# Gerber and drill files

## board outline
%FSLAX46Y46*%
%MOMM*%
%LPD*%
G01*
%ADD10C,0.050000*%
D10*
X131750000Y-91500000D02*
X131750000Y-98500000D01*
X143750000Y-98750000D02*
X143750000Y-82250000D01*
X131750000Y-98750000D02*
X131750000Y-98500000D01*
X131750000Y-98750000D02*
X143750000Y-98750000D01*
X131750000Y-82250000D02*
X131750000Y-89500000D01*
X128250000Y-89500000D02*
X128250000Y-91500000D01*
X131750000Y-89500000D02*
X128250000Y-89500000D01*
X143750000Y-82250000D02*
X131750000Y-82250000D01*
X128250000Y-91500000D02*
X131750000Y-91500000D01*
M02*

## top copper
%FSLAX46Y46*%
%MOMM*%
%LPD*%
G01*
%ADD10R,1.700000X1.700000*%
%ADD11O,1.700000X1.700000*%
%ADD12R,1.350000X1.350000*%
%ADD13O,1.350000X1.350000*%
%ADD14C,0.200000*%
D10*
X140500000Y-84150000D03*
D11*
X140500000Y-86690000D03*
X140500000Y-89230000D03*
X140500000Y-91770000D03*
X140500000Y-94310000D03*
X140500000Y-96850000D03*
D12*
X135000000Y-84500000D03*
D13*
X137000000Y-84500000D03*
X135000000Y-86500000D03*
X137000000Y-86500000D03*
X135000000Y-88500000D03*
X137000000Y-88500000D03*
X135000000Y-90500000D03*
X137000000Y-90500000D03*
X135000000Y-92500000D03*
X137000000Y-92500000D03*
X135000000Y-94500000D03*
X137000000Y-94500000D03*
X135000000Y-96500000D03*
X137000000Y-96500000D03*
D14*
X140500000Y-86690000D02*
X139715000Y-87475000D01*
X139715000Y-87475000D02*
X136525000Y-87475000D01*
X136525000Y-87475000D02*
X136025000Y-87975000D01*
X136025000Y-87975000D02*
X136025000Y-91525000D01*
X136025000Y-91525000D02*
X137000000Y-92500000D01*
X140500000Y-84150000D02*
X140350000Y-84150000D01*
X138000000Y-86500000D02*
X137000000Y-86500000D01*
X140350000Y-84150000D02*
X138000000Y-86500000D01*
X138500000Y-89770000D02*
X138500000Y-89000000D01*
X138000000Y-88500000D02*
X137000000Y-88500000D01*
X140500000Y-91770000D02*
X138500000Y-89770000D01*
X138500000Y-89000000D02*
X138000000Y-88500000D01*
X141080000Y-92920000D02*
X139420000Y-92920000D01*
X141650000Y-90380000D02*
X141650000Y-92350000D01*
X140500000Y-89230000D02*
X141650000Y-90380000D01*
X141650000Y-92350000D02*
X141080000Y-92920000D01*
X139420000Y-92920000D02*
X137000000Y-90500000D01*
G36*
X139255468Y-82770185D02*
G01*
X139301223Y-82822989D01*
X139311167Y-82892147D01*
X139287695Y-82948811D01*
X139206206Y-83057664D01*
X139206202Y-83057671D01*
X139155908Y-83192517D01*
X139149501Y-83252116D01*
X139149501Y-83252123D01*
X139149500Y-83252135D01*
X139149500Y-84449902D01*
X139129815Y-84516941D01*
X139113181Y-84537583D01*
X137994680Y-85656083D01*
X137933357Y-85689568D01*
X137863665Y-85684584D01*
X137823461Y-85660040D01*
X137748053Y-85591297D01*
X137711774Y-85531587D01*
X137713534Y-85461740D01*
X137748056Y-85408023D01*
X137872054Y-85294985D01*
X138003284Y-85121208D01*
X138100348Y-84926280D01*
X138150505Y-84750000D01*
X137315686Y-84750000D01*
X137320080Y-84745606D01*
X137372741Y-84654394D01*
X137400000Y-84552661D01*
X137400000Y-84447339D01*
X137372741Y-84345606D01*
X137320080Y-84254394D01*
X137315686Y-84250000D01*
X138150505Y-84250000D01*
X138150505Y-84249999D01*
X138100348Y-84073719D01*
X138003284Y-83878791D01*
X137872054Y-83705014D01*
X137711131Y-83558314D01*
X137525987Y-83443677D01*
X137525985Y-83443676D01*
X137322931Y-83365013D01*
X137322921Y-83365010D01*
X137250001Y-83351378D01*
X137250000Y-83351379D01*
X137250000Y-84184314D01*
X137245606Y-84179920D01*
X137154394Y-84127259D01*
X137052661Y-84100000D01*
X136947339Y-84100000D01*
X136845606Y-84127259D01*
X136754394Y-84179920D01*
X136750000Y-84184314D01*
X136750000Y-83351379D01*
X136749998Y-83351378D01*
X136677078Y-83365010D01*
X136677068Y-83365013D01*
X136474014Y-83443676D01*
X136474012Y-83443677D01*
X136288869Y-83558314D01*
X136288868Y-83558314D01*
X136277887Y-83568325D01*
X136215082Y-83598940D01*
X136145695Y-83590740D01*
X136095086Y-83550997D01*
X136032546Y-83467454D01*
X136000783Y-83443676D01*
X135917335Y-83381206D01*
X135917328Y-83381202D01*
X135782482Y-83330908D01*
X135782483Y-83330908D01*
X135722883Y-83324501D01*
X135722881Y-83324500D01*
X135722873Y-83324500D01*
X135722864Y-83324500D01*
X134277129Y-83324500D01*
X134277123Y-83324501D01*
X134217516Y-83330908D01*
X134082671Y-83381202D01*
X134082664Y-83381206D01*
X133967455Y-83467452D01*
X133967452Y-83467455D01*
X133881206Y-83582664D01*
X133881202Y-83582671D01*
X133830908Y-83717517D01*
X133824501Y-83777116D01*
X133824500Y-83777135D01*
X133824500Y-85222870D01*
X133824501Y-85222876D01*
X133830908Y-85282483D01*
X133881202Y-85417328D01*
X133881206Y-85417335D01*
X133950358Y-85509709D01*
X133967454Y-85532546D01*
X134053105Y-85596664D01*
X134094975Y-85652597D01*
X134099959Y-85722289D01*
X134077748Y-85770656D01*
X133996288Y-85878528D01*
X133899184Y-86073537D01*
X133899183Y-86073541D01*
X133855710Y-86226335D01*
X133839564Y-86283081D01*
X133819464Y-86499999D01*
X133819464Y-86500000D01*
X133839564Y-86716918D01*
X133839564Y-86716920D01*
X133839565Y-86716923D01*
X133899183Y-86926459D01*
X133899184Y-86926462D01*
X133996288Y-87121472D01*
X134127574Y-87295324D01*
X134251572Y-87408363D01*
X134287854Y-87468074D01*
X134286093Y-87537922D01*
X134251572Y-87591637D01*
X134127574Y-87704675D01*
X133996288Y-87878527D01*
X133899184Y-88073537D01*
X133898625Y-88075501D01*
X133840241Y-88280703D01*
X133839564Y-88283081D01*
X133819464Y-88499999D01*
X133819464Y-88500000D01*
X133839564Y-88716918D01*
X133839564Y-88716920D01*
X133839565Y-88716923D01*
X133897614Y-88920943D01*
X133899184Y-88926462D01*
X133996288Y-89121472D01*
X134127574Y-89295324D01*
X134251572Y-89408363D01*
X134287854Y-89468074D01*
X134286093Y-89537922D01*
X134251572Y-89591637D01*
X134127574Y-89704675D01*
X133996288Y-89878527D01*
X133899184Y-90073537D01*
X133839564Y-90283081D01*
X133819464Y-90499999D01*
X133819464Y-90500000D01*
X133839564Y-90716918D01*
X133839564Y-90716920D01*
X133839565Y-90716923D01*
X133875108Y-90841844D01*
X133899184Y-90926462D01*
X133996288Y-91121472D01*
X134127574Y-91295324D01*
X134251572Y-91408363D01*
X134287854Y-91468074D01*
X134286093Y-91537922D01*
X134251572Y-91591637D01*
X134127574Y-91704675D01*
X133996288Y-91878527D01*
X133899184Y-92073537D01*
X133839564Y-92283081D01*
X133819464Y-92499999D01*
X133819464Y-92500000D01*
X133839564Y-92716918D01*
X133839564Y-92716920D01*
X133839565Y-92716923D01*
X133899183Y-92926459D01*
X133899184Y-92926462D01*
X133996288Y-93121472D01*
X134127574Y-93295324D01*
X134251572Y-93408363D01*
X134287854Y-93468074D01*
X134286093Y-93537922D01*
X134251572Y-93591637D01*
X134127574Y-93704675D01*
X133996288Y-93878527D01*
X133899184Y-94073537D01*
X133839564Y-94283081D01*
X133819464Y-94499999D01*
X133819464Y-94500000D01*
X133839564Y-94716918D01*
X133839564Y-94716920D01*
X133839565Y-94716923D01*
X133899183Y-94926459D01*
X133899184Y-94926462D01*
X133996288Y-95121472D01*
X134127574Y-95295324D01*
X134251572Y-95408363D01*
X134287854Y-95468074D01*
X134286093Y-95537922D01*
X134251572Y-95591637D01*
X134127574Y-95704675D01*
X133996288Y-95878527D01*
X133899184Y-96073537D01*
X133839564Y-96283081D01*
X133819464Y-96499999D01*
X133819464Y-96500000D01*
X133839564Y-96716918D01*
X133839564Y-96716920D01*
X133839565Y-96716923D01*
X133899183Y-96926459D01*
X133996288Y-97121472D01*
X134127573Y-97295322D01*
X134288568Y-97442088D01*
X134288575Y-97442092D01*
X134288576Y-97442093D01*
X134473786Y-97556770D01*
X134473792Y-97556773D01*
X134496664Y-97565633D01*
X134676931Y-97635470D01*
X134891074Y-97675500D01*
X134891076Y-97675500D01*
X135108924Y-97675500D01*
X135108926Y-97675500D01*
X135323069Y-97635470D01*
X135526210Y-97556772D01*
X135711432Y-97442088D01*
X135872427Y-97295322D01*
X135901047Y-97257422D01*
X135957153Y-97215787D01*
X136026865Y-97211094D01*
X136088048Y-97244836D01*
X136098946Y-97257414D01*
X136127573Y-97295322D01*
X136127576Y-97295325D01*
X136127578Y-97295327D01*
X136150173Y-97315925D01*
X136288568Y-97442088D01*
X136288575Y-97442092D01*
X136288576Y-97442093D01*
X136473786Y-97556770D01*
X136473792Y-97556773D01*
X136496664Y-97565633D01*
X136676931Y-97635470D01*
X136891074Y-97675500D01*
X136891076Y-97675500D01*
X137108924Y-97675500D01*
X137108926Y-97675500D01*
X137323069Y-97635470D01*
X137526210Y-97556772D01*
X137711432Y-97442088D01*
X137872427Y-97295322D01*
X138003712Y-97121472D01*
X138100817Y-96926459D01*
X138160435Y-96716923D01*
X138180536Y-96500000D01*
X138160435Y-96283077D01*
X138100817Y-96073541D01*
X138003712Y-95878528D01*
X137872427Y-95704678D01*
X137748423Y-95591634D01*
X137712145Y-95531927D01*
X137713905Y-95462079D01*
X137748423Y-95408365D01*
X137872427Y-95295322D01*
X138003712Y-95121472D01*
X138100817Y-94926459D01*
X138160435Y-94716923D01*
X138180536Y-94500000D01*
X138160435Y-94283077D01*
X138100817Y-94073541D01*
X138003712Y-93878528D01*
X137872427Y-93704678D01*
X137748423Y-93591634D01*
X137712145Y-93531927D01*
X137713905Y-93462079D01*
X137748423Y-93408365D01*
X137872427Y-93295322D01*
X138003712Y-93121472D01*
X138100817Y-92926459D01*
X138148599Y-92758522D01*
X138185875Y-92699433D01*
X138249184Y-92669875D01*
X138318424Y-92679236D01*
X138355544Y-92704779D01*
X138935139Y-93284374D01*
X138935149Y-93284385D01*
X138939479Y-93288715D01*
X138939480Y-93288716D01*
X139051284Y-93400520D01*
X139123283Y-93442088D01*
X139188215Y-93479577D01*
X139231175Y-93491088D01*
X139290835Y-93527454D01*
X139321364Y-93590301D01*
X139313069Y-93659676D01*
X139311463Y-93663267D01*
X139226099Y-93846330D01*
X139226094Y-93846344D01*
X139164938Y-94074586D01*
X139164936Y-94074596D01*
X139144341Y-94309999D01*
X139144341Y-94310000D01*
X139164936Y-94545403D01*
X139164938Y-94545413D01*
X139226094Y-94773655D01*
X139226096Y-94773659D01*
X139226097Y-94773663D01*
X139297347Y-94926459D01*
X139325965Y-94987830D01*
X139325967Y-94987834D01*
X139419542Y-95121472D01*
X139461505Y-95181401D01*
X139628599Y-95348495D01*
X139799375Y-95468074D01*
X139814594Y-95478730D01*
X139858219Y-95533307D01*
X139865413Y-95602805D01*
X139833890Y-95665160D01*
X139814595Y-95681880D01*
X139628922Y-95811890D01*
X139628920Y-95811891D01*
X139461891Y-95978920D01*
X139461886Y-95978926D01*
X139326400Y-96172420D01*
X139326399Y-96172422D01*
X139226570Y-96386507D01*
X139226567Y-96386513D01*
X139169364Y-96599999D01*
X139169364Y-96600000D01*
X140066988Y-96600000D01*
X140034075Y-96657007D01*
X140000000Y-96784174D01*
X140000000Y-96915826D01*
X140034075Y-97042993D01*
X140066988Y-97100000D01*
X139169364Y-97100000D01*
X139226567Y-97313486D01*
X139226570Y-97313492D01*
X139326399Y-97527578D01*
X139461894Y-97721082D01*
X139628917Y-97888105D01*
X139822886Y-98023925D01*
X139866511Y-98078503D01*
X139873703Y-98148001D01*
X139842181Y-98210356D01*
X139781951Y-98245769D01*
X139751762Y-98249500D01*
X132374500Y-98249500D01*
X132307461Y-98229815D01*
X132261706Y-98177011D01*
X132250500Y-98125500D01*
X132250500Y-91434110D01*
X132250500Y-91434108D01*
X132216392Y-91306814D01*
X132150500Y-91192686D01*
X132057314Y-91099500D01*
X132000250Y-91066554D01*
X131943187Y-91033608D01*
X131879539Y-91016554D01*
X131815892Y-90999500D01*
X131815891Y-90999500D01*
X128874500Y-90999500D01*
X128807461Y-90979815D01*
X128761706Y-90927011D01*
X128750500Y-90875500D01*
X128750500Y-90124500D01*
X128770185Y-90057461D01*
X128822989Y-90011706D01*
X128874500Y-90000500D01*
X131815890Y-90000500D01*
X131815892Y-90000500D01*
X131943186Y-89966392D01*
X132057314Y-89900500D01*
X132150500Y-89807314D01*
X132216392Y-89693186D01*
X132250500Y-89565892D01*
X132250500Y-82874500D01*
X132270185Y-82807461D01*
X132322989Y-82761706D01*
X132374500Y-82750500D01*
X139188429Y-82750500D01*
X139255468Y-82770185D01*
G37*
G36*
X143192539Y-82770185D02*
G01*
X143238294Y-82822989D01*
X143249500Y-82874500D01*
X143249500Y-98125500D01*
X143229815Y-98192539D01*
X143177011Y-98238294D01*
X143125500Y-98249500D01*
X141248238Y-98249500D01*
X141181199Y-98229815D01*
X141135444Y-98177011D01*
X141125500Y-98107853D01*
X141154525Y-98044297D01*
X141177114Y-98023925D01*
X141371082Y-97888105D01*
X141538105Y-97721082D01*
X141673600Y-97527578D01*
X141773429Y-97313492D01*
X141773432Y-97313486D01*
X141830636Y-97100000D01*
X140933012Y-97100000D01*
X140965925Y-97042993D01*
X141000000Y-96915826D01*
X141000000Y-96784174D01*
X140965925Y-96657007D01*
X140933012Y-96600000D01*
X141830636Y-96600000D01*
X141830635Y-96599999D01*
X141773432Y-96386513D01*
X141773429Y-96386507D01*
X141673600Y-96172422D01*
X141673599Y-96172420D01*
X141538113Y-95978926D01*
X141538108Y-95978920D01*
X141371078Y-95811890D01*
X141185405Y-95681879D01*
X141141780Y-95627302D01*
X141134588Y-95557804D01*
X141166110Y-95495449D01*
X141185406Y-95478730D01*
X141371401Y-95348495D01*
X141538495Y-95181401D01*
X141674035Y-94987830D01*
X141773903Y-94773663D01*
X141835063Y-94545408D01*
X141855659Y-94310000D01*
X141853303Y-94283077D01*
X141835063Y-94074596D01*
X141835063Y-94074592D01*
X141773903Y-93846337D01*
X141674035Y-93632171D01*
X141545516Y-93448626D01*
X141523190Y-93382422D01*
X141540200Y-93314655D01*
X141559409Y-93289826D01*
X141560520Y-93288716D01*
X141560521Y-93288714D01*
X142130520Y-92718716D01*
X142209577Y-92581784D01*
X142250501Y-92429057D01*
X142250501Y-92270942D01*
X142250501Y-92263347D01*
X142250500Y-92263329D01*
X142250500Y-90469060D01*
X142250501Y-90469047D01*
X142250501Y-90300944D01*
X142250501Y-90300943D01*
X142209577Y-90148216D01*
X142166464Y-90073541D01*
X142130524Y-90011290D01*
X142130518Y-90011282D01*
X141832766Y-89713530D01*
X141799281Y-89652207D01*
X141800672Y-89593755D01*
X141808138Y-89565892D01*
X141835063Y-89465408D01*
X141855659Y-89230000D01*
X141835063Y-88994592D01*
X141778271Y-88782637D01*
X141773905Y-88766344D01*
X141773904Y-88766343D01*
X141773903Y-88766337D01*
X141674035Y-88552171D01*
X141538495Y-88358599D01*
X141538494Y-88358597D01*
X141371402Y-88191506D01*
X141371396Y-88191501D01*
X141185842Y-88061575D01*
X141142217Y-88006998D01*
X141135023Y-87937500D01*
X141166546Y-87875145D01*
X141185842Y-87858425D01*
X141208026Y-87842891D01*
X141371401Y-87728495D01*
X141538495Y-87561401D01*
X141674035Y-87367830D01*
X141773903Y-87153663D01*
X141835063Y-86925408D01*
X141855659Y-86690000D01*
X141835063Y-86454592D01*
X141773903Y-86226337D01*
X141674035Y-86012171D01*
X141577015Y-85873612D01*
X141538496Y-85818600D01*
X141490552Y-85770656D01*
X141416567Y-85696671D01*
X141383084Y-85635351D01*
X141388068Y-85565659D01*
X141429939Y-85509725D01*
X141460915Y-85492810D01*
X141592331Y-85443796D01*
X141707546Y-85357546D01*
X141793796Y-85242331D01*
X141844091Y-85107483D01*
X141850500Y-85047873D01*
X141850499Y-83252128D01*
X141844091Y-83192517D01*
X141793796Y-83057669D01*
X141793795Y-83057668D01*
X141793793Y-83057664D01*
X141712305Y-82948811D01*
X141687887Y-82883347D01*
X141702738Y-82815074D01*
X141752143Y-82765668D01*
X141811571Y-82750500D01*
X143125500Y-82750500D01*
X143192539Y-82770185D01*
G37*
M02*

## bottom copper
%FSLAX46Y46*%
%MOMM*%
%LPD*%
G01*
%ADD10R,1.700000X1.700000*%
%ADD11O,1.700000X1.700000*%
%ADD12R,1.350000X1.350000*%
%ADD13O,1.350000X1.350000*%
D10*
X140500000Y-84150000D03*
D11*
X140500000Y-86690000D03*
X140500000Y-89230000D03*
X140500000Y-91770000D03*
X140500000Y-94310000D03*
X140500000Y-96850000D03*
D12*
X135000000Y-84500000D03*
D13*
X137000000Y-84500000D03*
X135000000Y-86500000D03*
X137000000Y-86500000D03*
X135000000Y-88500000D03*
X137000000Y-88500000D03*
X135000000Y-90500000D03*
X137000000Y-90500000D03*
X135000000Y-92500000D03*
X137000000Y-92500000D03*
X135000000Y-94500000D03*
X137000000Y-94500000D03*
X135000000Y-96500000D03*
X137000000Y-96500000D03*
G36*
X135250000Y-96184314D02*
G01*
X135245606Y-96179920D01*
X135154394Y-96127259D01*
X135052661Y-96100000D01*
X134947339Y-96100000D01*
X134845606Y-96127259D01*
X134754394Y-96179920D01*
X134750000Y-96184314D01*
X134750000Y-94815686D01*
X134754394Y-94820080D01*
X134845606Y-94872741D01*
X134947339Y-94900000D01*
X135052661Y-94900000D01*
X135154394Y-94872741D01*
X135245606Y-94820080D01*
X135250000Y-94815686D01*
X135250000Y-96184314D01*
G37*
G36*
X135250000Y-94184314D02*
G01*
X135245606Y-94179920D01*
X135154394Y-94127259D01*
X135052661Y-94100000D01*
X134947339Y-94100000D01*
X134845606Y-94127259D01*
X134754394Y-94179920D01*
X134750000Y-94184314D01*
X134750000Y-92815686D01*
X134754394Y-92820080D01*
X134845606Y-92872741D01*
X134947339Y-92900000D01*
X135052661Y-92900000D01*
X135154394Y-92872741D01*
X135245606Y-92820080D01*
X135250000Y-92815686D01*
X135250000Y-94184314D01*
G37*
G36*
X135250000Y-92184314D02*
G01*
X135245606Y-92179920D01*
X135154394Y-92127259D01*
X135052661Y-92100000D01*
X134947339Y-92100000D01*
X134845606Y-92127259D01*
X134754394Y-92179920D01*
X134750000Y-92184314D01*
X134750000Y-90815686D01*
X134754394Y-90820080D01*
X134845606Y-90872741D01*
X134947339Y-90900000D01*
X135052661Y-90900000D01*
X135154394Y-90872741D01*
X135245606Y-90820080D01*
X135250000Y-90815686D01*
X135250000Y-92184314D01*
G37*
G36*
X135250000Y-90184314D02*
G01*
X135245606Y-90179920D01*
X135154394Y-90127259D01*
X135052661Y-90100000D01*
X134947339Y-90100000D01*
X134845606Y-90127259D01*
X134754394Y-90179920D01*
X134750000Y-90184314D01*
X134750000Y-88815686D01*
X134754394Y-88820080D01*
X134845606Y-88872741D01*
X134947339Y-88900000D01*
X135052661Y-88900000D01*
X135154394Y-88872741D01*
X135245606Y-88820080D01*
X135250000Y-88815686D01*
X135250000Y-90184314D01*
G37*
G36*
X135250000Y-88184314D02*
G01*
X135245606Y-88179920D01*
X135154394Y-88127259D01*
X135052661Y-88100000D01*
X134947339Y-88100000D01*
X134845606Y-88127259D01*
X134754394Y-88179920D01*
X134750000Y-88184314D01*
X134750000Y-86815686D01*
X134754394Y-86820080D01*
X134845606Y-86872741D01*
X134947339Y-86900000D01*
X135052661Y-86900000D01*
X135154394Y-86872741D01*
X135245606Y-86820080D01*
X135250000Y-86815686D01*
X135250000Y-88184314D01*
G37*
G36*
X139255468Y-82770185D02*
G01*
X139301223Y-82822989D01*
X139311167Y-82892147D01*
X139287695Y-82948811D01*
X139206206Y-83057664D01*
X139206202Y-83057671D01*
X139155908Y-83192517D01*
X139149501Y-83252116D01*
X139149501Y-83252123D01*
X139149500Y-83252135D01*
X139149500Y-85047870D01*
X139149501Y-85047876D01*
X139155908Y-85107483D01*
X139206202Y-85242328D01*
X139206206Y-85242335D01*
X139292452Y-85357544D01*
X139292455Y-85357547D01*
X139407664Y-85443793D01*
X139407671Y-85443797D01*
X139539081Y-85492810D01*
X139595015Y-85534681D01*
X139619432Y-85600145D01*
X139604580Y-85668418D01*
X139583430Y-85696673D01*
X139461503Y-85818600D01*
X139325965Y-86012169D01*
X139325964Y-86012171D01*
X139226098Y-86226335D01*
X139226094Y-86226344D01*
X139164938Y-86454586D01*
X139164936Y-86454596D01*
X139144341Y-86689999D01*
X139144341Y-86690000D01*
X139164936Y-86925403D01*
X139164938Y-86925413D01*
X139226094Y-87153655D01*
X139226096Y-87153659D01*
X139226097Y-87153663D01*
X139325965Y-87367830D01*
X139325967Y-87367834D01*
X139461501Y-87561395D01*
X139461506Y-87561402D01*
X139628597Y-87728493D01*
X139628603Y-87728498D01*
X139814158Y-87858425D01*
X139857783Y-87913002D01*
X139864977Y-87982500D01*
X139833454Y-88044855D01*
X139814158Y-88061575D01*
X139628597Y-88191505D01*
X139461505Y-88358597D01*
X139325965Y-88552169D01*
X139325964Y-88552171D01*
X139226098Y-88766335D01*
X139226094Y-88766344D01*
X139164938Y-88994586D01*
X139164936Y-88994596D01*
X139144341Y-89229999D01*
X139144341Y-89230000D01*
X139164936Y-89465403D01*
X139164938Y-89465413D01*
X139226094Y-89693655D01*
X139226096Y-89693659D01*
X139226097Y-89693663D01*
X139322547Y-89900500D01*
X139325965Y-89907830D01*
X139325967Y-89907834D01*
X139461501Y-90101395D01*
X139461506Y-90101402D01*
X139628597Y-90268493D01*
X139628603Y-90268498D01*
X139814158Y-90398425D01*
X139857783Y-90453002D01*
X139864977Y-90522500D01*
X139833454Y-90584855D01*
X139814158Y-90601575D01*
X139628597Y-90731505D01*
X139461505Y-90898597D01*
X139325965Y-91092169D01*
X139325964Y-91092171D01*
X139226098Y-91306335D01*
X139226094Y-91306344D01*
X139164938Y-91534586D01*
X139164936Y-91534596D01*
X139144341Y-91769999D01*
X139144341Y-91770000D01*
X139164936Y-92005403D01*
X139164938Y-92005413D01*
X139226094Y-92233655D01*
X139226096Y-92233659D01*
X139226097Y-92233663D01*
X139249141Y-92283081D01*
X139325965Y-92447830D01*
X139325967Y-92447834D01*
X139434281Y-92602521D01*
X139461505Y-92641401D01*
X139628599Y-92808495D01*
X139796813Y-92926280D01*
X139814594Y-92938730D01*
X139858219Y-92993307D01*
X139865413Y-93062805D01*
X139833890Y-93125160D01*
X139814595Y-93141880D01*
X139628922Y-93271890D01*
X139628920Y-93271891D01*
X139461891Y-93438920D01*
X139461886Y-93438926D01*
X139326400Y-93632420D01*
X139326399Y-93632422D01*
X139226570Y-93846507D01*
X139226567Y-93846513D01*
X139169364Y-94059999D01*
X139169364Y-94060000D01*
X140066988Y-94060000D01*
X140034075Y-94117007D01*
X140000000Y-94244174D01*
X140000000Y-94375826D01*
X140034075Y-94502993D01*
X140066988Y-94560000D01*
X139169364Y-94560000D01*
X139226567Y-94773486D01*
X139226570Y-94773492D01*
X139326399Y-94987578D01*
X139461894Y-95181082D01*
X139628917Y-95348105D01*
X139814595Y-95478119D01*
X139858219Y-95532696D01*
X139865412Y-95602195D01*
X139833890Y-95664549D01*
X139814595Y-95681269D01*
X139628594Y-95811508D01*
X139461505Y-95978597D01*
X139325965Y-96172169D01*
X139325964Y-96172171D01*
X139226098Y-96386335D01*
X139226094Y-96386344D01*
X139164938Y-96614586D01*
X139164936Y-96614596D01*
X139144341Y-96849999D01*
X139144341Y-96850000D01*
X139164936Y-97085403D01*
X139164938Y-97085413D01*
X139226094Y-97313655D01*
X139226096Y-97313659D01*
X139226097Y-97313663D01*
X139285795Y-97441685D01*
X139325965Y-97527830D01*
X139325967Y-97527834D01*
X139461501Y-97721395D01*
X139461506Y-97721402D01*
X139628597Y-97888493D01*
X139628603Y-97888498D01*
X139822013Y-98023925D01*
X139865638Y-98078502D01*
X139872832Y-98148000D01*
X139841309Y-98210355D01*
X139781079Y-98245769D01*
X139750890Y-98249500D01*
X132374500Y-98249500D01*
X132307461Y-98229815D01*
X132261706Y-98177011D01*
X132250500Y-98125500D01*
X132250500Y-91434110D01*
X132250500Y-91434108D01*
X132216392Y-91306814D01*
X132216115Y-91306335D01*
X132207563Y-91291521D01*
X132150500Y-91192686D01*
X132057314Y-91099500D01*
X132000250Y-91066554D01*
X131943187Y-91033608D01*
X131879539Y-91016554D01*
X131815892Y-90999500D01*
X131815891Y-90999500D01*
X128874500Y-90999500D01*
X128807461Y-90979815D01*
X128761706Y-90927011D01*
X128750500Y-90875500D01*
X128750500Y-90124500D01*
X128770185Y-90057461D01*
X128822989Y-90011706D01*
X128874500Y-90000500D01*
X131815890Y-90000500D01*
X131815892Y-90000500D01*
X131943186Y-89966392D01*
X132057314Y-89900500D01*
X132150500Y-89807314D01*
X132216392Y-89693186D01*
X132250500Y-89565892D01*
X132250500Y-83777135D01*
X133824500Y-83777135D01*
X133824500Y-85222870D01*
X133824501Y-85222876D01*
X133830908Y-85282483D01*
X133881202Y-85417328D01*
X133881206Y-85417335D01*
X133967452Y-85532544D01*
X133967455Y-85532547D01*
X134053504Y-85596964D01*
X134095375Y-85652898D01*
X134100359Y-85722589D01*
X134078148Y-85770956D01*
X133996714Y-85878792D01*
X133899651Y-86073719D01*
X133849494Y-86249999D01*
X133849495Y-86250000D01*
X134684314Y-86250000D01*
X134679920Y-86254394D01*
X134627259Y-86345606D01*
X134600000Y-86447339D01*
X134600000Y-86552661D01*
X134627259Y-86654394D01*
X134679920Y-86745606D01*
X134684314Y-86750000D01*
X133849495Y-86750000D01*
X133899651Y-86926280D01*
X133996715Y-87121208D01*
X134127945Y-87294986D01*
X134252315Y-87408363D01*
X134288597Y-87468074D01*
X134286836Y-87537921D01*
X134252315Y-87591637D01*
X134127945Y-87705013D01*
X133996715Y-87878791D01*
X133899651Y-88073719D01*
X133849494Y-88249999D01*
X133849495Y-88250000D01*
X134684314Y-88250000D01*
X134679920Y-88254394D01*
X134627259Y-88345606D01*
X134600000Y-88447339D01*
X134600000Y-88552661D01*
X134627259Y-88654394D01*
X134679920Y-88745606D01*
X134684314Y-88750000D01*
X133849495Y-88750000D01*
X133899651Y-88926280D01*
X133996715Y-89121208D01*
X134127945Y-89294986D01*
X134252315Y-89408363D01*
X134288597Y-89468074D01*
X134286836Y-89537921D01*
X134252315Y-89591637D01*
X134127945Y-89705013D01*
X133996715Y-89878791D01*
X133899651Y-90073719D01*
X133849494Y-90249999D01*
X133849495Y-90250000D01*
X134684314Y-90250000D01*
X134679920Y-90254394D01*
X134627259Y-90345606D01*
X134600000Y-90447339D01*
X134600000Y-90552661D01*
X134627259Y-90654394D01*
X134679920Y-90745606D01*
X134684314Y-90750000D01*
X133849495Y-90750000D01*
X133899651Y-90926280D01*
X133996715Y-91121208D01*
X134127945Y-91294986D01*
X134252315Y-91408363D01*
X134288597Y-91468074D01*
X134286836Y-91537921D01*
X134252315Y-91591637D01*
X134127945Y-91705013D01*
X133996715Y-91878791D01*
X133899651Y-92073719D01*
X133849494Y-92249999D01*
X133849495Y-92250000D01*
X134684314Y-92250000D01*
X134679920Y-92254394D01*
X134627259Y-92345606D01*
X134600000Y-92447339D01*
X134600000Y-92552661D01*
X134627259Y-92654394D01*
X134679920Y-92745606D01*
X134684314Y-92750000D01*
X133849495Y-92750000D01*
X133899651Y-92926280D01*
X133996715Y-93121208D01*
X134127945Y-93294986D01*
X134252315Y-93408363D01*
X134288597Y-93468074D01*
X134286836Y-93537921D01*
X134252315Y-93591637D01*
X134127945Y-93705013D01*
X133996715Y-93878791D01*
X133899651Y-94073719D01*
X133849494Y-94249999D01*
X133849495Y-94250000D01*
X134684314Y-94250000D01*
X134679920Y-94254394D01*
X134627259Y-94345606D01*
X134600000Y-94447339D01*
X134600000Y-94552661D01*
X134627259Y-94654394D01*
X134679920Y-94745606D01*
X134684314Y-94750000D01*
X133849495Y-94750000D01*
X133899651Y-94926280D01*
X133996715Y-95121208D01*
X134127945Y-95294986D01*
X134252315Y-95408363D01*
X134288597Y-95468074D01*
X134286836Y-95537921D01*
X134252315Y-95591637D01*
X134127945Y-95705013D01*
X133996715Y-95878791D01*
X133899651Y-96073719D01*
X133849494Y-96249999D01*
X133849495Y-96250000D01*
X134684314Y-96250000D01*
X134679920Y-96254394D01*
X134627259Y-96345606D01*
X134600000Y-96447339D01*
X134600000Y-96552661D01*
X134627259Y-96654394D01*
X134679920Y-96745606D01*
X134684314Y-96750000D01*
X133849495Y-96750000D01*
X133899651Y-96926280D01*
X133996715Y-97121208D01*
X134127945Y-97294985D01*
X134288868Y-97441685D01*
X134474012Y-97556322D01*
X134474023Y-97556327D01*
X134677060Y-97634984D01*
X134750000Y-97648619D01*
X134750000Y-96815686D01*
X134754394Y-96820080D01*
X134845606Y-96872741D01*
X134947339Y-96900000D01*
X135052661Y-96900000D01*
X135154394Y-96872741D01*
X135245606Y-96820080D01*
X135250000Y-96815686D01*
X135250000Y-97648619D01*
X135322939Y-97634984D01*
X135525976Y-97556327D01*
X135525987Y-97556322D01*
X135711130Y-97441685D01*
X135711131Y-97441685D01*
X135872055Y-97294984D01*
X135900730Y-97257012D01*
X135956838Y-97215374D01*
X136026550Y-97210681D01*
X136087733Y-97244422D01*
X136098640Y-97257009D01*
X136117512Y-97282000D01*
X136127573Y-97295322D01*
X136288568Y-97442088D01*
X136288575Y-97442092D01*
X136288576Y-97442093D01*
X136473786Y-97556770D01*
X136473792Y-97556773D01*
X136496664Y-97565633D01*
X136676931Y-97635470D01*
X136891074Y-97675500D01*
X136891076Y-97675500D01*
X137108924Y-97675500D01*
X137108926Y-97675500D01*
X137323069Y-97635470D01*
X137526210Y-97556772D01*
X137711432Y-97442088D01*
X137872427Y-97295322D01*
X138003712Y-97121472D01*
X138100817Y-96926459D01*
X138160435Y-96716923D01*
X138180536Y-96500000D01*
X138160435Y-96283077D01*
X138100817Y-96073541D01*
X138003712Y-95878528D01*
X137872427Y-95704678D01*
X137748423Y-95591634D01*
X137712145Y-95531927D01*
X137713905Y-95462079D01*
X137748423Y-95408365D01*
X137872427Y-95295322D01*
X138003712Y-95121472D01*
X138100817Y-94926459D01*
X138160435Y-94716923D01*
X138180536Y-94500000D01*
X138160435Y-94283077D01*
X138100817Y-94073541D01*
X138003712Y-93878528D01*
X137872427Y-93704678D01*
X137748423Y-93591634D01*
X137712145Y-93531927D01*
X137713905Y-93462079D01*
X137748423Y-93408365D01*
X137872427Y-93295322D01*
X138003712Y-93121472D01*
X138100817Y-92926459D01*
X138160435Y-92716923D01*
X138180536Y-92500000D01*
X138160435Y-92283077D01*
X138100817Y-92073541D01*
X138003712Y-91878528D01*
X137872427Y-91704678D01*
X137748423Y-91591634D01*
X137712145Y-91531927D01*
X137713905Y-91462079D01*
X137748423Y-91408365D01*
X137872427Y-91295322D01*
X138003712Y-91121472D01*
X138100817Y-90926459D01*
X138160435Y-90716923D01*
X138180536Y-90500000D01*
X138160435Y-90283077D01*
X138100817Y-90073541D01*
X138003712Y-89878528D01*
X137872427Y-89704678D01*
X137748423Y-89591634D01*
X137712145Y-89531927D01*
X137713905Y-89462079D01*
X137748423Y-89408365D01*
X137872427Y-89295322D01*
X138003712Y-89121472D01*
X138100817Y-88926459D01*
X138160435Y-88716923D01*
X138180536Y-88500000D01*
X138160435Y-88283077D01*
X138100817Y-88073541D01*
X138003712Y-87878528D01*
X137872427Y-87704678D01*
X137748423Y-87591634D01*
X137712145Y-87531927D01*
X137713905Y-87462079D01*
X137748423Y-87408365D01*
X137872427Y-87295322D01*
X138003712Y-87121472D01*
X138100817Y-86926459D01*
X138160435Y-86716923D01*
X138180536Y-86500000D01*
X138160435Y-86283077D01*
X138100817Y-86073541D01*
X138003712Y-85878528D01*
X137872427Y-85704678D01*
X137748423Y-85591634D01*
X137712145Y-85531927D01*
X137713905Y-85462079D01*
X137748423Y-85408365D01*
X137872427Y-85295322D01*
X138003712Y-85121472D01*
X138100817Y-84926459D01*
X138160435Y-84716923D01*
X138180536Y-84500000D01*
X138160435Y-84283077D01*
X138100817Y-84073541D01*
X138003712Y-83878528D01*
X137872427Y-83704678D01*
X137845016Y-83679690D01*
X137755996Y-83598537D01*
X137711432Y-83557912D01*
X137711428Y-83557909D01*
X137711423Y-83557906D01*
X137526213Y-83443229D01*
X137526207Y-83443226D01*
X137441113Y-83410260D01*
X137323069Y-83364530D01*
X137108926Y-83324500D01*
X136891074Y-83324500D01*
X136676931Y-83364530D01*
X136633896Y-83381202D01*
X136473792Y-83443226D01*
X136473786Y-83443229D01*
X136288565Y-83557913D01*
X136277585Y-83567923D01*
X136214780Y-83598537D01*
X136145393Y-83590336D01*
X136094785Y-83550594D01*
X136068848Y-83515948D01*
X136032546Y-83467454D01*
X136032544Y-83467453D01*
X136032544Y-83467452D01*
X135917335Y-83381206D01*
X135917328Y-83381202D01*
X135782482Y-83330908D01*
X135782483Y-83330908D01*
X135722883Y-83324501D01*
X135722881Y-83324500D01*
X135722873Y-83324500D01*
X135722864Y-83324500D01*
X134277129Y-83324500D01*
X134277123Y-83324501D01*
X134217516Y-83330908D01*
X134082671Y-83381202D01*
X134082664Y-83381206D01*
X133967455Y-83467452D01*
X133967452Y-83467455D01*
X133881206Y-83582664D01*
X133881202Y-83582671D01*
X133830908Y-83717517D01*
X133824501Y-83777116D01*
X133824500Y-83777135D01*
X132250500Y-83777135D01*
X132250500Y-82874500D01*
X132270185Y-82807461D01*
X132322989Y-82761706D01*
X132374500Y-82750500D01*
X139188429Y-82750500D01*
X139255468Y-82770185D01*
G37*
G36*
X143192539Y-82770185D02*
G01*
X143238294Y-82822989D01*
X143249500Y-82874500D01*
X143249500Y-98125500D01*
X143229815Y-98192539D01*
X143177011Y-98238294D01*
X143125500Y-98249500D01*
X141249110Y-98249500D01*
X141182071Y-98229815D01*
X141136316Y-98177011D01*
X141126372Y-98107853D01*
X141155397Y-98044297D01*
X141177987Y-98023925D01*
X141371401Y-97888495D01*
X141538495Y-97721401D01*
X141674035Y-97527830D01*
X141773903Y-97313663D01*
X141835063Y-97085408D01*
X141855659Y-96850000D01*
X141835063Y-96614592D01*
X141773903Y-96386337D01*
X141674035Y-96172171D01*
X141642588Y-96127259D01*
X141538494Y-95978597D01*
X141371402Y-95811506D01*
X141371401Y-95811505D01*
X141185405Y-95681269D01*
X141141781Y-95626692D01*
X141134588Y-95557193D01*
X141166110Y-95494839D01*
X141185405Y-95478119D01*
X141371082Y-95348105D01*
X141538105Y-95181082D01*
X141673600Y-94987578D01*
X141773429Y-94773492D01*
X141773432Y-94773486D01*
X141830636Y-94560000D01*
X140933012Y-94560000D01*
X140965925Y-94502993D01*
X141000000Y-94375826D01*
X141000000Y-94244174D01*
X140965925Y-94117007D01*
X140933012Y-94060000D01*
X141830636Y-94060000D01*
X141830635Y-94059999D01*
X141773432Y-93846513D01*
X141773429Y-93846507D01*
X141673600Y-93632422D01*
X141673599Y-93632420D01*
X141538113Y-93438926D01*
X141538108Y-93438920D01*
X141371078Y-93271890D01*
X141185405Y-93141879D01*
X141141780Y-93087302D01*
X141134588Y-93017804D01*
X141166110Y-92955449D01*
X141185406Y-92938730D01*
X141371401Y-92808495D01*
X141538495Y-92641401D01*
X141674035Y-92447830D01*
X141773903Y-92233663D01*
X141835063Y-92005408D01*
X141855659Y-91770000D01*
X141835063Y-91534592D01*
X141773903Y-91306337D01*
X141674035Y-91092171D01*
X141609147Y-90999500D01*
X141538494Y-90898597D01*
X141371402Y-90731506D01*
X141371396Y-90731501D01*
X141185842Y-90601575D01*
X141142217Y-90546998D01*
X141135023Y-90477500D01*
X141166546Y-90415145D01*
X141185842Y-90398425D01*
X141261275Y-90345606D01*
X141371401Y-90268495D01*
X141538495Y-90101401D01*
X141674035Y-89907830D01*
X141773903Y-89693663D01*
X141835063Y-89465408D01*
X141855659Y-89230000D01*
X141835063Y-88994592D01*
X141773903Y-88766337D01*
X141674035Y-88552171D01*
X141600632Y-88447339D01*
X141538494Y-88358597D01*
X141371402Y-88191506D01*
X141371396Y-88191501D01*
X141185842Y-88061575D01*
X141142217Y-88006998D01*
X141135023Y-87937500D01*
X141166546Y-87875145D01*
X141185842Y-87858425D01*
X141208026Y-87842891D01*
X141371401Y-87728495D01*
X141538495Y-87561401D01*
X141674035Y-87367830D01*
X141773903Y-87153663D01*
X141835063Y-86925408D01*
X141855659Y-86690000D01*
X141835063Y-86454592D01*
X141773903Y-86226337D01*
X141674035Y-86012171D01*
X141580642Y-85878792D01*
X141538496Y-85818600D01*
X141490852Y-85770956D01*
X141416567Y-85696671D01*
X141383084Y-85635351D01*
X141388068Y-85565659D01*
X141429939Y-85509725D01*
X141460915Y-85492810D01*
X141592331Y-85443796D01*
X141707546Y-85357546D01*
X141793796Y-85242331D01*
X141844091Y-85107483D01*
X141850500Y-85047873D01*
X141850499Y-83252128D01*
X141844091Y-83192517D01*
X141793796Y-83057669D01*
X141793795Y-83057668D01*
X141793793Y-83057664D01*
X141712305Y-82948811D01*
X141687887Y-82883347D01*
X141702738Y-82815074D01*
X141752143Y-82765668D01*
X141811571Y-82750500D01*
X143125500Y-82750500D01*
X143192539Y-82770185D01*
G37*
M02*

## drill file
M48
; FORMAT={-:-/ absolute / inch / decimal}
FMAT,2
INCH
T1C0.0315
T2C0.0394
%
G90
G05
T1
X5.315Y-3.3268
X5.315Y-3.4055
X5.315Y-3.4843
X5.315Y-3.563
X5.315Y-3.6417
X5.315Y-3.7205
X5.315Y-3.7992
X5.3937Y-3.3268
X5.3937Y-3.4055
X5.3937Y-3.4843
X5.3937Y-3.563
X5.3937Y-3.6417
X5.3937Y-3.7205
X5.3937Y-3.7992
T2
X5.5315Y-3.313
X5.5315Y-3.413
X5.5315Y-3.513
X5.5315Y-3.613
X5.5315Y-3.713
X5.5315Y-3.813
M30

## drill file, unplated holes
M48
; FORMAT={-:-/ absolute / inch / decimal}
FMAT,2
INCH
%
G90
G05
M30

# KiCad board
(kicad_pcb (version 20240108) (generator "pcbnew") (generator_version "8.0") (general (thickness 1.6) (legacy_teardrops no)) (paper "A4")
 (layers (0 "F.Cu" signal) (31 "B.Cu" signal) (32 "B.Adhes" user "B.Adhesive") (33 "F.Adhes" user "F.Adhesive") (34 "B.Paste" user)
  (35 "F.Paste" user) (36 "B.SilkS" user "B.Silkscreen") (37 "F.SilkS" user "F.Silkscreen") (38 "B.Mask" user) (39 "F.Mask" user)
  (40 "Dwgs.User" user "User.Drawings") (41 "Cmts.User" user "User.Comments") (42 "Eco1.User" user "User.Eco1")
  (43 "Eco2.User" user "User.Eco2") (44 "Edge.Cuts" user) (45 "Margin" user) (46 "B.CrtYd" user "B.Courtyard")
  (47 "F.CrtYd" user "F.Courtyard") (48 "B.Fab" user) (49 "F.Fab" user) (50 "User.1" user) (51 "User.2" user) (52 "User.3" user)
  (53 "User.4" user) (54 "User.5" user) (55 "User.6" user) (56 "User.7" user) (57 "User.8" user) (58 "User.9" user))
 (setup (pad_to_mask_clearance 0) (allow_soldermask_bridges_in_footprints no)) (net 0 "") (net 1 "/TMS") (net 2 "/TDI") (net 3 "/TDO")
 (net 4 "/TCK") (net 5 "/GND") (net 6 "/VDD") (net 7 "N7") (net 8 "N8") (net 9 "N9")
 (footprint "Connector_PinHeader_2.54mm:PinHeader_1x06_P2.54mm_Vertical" (layer "F.Cu") (at 140.5 84.15)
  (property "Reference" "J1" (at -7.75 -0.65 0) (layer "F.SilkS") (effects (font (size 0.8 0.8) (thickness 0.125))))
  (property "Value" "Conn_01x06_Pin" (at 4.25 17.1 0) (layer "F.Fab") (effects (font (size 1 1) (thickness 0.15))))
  (pad "1" thru_hole rect (at 0 0) (size 1.7 1.7) (drill 1) (layers "*.Cu" "*.Mask") (remove_unused_layers no) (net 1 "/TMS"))
  (pad "2" thru_hole oval (at 0 2.54) (size 1.7 1.7) (drill 1) (layers "*.Cu" "*.Mask") (remove_unused_layers no) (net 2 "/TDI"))
  (pad "3" thru_hole oval (at 0 5.08) (size 1.7 1.7) (drill 1) (layers "*.Cu" "*.Mask") (remove_unused_layers no) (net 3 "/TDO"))
  (pad "4" thru_hole oval (at 0 7.62) (size 1.7 1.7) (drill 1) (layers "*.Cu" "*.Mask") (remove_unused_layers no) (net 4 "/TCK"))
  (pad "5" thru_hole oval (at 0 10.16) (size 1.7 1.7) (drill 1) (layers "*.Cu" "*.Mask") (remove_unused_layers no) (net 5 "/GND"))
  (pad "6" thru_hole oval (at 0 12.7) (size 1.7 1.7) (drill 1) (layers "*.Cu" "*.Mask") (remove_unused_layers no) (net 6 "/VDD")))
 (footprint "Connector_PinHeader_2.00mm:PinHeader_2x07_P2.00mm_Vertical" (layer "F.Cu") (at 135 84.5)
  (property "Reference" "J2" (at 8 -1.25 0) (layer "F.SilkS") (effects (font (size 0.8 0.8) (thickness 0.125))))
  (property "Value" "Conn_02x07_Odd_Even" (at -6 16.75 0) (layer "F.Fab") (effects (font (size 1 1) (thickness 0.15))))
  (pad "1" thru_hole rect (at 0 0) (size 1.35 1.35) (drill 0.8) (layers "*.Cu" "*.Mask") (remove_unused_layers no) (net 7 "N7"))
  (pad "2" thru_hole oval (at 2 0) (size 1.35 1.35) (drill 0.8) (layers "*.Cu" "*.Mask") (remove_unused_layers no) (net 6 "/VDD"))
  (pad "3" thru_hole oval (at 0 2) (size 1.35 1.35) (drill 0.8) (layers "*.Cu" "*.Mask") (remove_unused_layers no) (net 5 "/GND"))
  (pad "4" thru_hole oval (at 2 2) (size 1.35 1.35) (drill 0.8) (layers "*.Cu" "*.Mask") (remove_unused_layers no) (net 1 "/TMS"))
  (pad "5" thru_hole oval (at 0 4) (size 1.35 1.35) (drill 0.8) (layers "*.Cu" "*.Mask") (remove_unused_layers no) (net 5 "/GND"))
  (pad "6" thru_hole oval (at 2 4) (size 1.35 1.35) (drill 0.8) (layers "*.Cu" "*.Mask") (remove_unused_layers no) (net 4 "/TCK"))
  (pad "7" thru_hole oval (at 0 6) (size 1.35 1.35) (drill 0.8) (layers "*.Cu" "*.Mask") (remove_unused_layers no) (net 5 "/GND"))
  (pad "8" thru_hole oval (at 2 6) (size 1.35 1.35) (drill 0.8) (layers "*.Cu" "*.Mask") (remove_unused_layers no) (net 3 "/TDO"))
  (pad "9" thru_hole oval (at 0 8) (size 1.35 1.35) (drill 0.8) (layers "*.Cu" "*.Mask") (remove_unused_layers no) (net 5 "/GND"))
  (pad "10" thru_hole oval (at 2 8) (size 1.35 1.35) (drill 0.8) (layers "*.Cu" "*.Mask") (remove_unused_layers no) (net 2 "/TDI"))
  (pad "11" thru_hole oval (at 0 10) (size 1.35 1.35) (drill 0.8) (layers "*.Cu" "*.Mask") (remove_unused_layers no) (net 5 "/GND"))
  (pad "12" thru_hole oval (at 2 10) (size 1.35 1.35) (drill 0.8) (layers "*.Cu" "*.Mask") (remove_unused_layers no) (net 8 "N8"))
  (pad "13" thru_hole oval (at 0 12) (size 1.35 1.35) (drill 0.8) (layers "*.Cu" "*.Mask") (remove_unused_layers no) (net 5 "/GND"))
  (pad "14" thru_hole oval (at 2 12) (size 1.35 1.35) (drill 0.8) (layers "*.Cu" "*.Mask") (remove_unused_layers no) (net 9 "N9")))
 (gr_line (start 131.75 91.5) (end 131.75 98.5) (stroke (width 0.05) (type default)) (layer "Edge.Cuts"))
 (gr_line (start 143.75 98.75) (end 143.75 82.25) (stroke (width 0.05) (type default)) (layer "Edge.Cuts"))
 (gr_line (start 131.75 98.75) (end 131.75 98.5) (stroke (width 0.05) (type default)) (layer "Edge.Cuts"))
 (gr_line (start 131.75 98.75) (end 143.75 98.75) (stroke (width 0.05) (type default)) (layer "Edge.Cuts"))
 (gr_line (start 131.75 82.25) (end 131.75 89.5) (stroke (width 0.05) (type default)) (layer "Edge.Cuts"))
 (gr_line (start 128.25 89.5) (end 128.25 91.5) (stroke (width 0.05) (type default)) (layer "Edge.Cuts"))
 (gr_line (start 131.75 89.5) (end 128.25 89.5) (stroke (width 0.05) (type default)) (layer "Edge.Cuts"))
 (gr_line (start 143.75 82.25) (end 131.75 82.25) (stroke (width 0.05) (type default)) (layer "Edge.Cuts"))
 (gr_line (start 128.25 91.5) (end 131.75 91.5) (stroke (width 0.05) (type default)) (layer "Edge.Cuts"))
 (segment (start 140.5 86.69) (end 139.715 87.475) (width 0.2) (layer "F.Cu") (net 2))
 (segment (start 139.715 87.475) (end 136.525 87.475) (width 0.2) (layer "F.Cu") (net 2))
 (segment (start 136.525 87.475) (end 136.025 87.975) (width 0.2) (layer "F.Cu") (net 2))
 (segment (start 136.025 87.975) (end 136.025 91.525) (width 0.2) (layer "F.Cu") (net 2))
 (segment (start 136.025 91.525) (end 137 92.5) (width 0.2) (layer "F.Cu") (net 2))
 (segment (start 140.5 84.15) (end 140.35 84.15) (width 0.2) (layer "F.Cu") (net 1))
 (segment (start 138 86.5) (end 137 86.5) (width 0.2) (layer "F.Cu") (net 1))
 (segment (start 140.35 84.15) (end 138 86.5) (width 0.2) (layer "F.Cu") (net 1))
 (segment (start 138.5 89.77) (end 138.5 89) (width 0.2) (layer "F.Cu") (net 4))
 (segment (start 138 88.5) (end 137 88.5) (width 0.2) (layer "F.Cu") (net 4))
 (segment (start 140.5 91.77) (end 138.5 89.77) (width 0.2) (layer "F.Cu") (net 4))
 (segment (start 138.5 89) (end 138 88.5) (width 0.2) (layer "F.Cu") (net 4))
 (segment (start 141.08 92.92) (end 139.42 92.92) (width 0.2) (layer "F.Cu") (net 3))
 (segment (start 141.65 90.38) (end 141.65 92.35) (width 0.2) (layer "F.Cu") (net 3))
 (segment (start 140.5 89.23) (end 141.65 90.38) (width 0.2) (layer "F.Cu") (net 3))
 (segment (start 141.65 92.35) (end 141.08 92.92) (width 0.2) (layer "F.Cu") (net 3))
 (segment (start 139.42 92.92) (end 137 90.5) (width 0.2) (layer "F.Cu") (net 3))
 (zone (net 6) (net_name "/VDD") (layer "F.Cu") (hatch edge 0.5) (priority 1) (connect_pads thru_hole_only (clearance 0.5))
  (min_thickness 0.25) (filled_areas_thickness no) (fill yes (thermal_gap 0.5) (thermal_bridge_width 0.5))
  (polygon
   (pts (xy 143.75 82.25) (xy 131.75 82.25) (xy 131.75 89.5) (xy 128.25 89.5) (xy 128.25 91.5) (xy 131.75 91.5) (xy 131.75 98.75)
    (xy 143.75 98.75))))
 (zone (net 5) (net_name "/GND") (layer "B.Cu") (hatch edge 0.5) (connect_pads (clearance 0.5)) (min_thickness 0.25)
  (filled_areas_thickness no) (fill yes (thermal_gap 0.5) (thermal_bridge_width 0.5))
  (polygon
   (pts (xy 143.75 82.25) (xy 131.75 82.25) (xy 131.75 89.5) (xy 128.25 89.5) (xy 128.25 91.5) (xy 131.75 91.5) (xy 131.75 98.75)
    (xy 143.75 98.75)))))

